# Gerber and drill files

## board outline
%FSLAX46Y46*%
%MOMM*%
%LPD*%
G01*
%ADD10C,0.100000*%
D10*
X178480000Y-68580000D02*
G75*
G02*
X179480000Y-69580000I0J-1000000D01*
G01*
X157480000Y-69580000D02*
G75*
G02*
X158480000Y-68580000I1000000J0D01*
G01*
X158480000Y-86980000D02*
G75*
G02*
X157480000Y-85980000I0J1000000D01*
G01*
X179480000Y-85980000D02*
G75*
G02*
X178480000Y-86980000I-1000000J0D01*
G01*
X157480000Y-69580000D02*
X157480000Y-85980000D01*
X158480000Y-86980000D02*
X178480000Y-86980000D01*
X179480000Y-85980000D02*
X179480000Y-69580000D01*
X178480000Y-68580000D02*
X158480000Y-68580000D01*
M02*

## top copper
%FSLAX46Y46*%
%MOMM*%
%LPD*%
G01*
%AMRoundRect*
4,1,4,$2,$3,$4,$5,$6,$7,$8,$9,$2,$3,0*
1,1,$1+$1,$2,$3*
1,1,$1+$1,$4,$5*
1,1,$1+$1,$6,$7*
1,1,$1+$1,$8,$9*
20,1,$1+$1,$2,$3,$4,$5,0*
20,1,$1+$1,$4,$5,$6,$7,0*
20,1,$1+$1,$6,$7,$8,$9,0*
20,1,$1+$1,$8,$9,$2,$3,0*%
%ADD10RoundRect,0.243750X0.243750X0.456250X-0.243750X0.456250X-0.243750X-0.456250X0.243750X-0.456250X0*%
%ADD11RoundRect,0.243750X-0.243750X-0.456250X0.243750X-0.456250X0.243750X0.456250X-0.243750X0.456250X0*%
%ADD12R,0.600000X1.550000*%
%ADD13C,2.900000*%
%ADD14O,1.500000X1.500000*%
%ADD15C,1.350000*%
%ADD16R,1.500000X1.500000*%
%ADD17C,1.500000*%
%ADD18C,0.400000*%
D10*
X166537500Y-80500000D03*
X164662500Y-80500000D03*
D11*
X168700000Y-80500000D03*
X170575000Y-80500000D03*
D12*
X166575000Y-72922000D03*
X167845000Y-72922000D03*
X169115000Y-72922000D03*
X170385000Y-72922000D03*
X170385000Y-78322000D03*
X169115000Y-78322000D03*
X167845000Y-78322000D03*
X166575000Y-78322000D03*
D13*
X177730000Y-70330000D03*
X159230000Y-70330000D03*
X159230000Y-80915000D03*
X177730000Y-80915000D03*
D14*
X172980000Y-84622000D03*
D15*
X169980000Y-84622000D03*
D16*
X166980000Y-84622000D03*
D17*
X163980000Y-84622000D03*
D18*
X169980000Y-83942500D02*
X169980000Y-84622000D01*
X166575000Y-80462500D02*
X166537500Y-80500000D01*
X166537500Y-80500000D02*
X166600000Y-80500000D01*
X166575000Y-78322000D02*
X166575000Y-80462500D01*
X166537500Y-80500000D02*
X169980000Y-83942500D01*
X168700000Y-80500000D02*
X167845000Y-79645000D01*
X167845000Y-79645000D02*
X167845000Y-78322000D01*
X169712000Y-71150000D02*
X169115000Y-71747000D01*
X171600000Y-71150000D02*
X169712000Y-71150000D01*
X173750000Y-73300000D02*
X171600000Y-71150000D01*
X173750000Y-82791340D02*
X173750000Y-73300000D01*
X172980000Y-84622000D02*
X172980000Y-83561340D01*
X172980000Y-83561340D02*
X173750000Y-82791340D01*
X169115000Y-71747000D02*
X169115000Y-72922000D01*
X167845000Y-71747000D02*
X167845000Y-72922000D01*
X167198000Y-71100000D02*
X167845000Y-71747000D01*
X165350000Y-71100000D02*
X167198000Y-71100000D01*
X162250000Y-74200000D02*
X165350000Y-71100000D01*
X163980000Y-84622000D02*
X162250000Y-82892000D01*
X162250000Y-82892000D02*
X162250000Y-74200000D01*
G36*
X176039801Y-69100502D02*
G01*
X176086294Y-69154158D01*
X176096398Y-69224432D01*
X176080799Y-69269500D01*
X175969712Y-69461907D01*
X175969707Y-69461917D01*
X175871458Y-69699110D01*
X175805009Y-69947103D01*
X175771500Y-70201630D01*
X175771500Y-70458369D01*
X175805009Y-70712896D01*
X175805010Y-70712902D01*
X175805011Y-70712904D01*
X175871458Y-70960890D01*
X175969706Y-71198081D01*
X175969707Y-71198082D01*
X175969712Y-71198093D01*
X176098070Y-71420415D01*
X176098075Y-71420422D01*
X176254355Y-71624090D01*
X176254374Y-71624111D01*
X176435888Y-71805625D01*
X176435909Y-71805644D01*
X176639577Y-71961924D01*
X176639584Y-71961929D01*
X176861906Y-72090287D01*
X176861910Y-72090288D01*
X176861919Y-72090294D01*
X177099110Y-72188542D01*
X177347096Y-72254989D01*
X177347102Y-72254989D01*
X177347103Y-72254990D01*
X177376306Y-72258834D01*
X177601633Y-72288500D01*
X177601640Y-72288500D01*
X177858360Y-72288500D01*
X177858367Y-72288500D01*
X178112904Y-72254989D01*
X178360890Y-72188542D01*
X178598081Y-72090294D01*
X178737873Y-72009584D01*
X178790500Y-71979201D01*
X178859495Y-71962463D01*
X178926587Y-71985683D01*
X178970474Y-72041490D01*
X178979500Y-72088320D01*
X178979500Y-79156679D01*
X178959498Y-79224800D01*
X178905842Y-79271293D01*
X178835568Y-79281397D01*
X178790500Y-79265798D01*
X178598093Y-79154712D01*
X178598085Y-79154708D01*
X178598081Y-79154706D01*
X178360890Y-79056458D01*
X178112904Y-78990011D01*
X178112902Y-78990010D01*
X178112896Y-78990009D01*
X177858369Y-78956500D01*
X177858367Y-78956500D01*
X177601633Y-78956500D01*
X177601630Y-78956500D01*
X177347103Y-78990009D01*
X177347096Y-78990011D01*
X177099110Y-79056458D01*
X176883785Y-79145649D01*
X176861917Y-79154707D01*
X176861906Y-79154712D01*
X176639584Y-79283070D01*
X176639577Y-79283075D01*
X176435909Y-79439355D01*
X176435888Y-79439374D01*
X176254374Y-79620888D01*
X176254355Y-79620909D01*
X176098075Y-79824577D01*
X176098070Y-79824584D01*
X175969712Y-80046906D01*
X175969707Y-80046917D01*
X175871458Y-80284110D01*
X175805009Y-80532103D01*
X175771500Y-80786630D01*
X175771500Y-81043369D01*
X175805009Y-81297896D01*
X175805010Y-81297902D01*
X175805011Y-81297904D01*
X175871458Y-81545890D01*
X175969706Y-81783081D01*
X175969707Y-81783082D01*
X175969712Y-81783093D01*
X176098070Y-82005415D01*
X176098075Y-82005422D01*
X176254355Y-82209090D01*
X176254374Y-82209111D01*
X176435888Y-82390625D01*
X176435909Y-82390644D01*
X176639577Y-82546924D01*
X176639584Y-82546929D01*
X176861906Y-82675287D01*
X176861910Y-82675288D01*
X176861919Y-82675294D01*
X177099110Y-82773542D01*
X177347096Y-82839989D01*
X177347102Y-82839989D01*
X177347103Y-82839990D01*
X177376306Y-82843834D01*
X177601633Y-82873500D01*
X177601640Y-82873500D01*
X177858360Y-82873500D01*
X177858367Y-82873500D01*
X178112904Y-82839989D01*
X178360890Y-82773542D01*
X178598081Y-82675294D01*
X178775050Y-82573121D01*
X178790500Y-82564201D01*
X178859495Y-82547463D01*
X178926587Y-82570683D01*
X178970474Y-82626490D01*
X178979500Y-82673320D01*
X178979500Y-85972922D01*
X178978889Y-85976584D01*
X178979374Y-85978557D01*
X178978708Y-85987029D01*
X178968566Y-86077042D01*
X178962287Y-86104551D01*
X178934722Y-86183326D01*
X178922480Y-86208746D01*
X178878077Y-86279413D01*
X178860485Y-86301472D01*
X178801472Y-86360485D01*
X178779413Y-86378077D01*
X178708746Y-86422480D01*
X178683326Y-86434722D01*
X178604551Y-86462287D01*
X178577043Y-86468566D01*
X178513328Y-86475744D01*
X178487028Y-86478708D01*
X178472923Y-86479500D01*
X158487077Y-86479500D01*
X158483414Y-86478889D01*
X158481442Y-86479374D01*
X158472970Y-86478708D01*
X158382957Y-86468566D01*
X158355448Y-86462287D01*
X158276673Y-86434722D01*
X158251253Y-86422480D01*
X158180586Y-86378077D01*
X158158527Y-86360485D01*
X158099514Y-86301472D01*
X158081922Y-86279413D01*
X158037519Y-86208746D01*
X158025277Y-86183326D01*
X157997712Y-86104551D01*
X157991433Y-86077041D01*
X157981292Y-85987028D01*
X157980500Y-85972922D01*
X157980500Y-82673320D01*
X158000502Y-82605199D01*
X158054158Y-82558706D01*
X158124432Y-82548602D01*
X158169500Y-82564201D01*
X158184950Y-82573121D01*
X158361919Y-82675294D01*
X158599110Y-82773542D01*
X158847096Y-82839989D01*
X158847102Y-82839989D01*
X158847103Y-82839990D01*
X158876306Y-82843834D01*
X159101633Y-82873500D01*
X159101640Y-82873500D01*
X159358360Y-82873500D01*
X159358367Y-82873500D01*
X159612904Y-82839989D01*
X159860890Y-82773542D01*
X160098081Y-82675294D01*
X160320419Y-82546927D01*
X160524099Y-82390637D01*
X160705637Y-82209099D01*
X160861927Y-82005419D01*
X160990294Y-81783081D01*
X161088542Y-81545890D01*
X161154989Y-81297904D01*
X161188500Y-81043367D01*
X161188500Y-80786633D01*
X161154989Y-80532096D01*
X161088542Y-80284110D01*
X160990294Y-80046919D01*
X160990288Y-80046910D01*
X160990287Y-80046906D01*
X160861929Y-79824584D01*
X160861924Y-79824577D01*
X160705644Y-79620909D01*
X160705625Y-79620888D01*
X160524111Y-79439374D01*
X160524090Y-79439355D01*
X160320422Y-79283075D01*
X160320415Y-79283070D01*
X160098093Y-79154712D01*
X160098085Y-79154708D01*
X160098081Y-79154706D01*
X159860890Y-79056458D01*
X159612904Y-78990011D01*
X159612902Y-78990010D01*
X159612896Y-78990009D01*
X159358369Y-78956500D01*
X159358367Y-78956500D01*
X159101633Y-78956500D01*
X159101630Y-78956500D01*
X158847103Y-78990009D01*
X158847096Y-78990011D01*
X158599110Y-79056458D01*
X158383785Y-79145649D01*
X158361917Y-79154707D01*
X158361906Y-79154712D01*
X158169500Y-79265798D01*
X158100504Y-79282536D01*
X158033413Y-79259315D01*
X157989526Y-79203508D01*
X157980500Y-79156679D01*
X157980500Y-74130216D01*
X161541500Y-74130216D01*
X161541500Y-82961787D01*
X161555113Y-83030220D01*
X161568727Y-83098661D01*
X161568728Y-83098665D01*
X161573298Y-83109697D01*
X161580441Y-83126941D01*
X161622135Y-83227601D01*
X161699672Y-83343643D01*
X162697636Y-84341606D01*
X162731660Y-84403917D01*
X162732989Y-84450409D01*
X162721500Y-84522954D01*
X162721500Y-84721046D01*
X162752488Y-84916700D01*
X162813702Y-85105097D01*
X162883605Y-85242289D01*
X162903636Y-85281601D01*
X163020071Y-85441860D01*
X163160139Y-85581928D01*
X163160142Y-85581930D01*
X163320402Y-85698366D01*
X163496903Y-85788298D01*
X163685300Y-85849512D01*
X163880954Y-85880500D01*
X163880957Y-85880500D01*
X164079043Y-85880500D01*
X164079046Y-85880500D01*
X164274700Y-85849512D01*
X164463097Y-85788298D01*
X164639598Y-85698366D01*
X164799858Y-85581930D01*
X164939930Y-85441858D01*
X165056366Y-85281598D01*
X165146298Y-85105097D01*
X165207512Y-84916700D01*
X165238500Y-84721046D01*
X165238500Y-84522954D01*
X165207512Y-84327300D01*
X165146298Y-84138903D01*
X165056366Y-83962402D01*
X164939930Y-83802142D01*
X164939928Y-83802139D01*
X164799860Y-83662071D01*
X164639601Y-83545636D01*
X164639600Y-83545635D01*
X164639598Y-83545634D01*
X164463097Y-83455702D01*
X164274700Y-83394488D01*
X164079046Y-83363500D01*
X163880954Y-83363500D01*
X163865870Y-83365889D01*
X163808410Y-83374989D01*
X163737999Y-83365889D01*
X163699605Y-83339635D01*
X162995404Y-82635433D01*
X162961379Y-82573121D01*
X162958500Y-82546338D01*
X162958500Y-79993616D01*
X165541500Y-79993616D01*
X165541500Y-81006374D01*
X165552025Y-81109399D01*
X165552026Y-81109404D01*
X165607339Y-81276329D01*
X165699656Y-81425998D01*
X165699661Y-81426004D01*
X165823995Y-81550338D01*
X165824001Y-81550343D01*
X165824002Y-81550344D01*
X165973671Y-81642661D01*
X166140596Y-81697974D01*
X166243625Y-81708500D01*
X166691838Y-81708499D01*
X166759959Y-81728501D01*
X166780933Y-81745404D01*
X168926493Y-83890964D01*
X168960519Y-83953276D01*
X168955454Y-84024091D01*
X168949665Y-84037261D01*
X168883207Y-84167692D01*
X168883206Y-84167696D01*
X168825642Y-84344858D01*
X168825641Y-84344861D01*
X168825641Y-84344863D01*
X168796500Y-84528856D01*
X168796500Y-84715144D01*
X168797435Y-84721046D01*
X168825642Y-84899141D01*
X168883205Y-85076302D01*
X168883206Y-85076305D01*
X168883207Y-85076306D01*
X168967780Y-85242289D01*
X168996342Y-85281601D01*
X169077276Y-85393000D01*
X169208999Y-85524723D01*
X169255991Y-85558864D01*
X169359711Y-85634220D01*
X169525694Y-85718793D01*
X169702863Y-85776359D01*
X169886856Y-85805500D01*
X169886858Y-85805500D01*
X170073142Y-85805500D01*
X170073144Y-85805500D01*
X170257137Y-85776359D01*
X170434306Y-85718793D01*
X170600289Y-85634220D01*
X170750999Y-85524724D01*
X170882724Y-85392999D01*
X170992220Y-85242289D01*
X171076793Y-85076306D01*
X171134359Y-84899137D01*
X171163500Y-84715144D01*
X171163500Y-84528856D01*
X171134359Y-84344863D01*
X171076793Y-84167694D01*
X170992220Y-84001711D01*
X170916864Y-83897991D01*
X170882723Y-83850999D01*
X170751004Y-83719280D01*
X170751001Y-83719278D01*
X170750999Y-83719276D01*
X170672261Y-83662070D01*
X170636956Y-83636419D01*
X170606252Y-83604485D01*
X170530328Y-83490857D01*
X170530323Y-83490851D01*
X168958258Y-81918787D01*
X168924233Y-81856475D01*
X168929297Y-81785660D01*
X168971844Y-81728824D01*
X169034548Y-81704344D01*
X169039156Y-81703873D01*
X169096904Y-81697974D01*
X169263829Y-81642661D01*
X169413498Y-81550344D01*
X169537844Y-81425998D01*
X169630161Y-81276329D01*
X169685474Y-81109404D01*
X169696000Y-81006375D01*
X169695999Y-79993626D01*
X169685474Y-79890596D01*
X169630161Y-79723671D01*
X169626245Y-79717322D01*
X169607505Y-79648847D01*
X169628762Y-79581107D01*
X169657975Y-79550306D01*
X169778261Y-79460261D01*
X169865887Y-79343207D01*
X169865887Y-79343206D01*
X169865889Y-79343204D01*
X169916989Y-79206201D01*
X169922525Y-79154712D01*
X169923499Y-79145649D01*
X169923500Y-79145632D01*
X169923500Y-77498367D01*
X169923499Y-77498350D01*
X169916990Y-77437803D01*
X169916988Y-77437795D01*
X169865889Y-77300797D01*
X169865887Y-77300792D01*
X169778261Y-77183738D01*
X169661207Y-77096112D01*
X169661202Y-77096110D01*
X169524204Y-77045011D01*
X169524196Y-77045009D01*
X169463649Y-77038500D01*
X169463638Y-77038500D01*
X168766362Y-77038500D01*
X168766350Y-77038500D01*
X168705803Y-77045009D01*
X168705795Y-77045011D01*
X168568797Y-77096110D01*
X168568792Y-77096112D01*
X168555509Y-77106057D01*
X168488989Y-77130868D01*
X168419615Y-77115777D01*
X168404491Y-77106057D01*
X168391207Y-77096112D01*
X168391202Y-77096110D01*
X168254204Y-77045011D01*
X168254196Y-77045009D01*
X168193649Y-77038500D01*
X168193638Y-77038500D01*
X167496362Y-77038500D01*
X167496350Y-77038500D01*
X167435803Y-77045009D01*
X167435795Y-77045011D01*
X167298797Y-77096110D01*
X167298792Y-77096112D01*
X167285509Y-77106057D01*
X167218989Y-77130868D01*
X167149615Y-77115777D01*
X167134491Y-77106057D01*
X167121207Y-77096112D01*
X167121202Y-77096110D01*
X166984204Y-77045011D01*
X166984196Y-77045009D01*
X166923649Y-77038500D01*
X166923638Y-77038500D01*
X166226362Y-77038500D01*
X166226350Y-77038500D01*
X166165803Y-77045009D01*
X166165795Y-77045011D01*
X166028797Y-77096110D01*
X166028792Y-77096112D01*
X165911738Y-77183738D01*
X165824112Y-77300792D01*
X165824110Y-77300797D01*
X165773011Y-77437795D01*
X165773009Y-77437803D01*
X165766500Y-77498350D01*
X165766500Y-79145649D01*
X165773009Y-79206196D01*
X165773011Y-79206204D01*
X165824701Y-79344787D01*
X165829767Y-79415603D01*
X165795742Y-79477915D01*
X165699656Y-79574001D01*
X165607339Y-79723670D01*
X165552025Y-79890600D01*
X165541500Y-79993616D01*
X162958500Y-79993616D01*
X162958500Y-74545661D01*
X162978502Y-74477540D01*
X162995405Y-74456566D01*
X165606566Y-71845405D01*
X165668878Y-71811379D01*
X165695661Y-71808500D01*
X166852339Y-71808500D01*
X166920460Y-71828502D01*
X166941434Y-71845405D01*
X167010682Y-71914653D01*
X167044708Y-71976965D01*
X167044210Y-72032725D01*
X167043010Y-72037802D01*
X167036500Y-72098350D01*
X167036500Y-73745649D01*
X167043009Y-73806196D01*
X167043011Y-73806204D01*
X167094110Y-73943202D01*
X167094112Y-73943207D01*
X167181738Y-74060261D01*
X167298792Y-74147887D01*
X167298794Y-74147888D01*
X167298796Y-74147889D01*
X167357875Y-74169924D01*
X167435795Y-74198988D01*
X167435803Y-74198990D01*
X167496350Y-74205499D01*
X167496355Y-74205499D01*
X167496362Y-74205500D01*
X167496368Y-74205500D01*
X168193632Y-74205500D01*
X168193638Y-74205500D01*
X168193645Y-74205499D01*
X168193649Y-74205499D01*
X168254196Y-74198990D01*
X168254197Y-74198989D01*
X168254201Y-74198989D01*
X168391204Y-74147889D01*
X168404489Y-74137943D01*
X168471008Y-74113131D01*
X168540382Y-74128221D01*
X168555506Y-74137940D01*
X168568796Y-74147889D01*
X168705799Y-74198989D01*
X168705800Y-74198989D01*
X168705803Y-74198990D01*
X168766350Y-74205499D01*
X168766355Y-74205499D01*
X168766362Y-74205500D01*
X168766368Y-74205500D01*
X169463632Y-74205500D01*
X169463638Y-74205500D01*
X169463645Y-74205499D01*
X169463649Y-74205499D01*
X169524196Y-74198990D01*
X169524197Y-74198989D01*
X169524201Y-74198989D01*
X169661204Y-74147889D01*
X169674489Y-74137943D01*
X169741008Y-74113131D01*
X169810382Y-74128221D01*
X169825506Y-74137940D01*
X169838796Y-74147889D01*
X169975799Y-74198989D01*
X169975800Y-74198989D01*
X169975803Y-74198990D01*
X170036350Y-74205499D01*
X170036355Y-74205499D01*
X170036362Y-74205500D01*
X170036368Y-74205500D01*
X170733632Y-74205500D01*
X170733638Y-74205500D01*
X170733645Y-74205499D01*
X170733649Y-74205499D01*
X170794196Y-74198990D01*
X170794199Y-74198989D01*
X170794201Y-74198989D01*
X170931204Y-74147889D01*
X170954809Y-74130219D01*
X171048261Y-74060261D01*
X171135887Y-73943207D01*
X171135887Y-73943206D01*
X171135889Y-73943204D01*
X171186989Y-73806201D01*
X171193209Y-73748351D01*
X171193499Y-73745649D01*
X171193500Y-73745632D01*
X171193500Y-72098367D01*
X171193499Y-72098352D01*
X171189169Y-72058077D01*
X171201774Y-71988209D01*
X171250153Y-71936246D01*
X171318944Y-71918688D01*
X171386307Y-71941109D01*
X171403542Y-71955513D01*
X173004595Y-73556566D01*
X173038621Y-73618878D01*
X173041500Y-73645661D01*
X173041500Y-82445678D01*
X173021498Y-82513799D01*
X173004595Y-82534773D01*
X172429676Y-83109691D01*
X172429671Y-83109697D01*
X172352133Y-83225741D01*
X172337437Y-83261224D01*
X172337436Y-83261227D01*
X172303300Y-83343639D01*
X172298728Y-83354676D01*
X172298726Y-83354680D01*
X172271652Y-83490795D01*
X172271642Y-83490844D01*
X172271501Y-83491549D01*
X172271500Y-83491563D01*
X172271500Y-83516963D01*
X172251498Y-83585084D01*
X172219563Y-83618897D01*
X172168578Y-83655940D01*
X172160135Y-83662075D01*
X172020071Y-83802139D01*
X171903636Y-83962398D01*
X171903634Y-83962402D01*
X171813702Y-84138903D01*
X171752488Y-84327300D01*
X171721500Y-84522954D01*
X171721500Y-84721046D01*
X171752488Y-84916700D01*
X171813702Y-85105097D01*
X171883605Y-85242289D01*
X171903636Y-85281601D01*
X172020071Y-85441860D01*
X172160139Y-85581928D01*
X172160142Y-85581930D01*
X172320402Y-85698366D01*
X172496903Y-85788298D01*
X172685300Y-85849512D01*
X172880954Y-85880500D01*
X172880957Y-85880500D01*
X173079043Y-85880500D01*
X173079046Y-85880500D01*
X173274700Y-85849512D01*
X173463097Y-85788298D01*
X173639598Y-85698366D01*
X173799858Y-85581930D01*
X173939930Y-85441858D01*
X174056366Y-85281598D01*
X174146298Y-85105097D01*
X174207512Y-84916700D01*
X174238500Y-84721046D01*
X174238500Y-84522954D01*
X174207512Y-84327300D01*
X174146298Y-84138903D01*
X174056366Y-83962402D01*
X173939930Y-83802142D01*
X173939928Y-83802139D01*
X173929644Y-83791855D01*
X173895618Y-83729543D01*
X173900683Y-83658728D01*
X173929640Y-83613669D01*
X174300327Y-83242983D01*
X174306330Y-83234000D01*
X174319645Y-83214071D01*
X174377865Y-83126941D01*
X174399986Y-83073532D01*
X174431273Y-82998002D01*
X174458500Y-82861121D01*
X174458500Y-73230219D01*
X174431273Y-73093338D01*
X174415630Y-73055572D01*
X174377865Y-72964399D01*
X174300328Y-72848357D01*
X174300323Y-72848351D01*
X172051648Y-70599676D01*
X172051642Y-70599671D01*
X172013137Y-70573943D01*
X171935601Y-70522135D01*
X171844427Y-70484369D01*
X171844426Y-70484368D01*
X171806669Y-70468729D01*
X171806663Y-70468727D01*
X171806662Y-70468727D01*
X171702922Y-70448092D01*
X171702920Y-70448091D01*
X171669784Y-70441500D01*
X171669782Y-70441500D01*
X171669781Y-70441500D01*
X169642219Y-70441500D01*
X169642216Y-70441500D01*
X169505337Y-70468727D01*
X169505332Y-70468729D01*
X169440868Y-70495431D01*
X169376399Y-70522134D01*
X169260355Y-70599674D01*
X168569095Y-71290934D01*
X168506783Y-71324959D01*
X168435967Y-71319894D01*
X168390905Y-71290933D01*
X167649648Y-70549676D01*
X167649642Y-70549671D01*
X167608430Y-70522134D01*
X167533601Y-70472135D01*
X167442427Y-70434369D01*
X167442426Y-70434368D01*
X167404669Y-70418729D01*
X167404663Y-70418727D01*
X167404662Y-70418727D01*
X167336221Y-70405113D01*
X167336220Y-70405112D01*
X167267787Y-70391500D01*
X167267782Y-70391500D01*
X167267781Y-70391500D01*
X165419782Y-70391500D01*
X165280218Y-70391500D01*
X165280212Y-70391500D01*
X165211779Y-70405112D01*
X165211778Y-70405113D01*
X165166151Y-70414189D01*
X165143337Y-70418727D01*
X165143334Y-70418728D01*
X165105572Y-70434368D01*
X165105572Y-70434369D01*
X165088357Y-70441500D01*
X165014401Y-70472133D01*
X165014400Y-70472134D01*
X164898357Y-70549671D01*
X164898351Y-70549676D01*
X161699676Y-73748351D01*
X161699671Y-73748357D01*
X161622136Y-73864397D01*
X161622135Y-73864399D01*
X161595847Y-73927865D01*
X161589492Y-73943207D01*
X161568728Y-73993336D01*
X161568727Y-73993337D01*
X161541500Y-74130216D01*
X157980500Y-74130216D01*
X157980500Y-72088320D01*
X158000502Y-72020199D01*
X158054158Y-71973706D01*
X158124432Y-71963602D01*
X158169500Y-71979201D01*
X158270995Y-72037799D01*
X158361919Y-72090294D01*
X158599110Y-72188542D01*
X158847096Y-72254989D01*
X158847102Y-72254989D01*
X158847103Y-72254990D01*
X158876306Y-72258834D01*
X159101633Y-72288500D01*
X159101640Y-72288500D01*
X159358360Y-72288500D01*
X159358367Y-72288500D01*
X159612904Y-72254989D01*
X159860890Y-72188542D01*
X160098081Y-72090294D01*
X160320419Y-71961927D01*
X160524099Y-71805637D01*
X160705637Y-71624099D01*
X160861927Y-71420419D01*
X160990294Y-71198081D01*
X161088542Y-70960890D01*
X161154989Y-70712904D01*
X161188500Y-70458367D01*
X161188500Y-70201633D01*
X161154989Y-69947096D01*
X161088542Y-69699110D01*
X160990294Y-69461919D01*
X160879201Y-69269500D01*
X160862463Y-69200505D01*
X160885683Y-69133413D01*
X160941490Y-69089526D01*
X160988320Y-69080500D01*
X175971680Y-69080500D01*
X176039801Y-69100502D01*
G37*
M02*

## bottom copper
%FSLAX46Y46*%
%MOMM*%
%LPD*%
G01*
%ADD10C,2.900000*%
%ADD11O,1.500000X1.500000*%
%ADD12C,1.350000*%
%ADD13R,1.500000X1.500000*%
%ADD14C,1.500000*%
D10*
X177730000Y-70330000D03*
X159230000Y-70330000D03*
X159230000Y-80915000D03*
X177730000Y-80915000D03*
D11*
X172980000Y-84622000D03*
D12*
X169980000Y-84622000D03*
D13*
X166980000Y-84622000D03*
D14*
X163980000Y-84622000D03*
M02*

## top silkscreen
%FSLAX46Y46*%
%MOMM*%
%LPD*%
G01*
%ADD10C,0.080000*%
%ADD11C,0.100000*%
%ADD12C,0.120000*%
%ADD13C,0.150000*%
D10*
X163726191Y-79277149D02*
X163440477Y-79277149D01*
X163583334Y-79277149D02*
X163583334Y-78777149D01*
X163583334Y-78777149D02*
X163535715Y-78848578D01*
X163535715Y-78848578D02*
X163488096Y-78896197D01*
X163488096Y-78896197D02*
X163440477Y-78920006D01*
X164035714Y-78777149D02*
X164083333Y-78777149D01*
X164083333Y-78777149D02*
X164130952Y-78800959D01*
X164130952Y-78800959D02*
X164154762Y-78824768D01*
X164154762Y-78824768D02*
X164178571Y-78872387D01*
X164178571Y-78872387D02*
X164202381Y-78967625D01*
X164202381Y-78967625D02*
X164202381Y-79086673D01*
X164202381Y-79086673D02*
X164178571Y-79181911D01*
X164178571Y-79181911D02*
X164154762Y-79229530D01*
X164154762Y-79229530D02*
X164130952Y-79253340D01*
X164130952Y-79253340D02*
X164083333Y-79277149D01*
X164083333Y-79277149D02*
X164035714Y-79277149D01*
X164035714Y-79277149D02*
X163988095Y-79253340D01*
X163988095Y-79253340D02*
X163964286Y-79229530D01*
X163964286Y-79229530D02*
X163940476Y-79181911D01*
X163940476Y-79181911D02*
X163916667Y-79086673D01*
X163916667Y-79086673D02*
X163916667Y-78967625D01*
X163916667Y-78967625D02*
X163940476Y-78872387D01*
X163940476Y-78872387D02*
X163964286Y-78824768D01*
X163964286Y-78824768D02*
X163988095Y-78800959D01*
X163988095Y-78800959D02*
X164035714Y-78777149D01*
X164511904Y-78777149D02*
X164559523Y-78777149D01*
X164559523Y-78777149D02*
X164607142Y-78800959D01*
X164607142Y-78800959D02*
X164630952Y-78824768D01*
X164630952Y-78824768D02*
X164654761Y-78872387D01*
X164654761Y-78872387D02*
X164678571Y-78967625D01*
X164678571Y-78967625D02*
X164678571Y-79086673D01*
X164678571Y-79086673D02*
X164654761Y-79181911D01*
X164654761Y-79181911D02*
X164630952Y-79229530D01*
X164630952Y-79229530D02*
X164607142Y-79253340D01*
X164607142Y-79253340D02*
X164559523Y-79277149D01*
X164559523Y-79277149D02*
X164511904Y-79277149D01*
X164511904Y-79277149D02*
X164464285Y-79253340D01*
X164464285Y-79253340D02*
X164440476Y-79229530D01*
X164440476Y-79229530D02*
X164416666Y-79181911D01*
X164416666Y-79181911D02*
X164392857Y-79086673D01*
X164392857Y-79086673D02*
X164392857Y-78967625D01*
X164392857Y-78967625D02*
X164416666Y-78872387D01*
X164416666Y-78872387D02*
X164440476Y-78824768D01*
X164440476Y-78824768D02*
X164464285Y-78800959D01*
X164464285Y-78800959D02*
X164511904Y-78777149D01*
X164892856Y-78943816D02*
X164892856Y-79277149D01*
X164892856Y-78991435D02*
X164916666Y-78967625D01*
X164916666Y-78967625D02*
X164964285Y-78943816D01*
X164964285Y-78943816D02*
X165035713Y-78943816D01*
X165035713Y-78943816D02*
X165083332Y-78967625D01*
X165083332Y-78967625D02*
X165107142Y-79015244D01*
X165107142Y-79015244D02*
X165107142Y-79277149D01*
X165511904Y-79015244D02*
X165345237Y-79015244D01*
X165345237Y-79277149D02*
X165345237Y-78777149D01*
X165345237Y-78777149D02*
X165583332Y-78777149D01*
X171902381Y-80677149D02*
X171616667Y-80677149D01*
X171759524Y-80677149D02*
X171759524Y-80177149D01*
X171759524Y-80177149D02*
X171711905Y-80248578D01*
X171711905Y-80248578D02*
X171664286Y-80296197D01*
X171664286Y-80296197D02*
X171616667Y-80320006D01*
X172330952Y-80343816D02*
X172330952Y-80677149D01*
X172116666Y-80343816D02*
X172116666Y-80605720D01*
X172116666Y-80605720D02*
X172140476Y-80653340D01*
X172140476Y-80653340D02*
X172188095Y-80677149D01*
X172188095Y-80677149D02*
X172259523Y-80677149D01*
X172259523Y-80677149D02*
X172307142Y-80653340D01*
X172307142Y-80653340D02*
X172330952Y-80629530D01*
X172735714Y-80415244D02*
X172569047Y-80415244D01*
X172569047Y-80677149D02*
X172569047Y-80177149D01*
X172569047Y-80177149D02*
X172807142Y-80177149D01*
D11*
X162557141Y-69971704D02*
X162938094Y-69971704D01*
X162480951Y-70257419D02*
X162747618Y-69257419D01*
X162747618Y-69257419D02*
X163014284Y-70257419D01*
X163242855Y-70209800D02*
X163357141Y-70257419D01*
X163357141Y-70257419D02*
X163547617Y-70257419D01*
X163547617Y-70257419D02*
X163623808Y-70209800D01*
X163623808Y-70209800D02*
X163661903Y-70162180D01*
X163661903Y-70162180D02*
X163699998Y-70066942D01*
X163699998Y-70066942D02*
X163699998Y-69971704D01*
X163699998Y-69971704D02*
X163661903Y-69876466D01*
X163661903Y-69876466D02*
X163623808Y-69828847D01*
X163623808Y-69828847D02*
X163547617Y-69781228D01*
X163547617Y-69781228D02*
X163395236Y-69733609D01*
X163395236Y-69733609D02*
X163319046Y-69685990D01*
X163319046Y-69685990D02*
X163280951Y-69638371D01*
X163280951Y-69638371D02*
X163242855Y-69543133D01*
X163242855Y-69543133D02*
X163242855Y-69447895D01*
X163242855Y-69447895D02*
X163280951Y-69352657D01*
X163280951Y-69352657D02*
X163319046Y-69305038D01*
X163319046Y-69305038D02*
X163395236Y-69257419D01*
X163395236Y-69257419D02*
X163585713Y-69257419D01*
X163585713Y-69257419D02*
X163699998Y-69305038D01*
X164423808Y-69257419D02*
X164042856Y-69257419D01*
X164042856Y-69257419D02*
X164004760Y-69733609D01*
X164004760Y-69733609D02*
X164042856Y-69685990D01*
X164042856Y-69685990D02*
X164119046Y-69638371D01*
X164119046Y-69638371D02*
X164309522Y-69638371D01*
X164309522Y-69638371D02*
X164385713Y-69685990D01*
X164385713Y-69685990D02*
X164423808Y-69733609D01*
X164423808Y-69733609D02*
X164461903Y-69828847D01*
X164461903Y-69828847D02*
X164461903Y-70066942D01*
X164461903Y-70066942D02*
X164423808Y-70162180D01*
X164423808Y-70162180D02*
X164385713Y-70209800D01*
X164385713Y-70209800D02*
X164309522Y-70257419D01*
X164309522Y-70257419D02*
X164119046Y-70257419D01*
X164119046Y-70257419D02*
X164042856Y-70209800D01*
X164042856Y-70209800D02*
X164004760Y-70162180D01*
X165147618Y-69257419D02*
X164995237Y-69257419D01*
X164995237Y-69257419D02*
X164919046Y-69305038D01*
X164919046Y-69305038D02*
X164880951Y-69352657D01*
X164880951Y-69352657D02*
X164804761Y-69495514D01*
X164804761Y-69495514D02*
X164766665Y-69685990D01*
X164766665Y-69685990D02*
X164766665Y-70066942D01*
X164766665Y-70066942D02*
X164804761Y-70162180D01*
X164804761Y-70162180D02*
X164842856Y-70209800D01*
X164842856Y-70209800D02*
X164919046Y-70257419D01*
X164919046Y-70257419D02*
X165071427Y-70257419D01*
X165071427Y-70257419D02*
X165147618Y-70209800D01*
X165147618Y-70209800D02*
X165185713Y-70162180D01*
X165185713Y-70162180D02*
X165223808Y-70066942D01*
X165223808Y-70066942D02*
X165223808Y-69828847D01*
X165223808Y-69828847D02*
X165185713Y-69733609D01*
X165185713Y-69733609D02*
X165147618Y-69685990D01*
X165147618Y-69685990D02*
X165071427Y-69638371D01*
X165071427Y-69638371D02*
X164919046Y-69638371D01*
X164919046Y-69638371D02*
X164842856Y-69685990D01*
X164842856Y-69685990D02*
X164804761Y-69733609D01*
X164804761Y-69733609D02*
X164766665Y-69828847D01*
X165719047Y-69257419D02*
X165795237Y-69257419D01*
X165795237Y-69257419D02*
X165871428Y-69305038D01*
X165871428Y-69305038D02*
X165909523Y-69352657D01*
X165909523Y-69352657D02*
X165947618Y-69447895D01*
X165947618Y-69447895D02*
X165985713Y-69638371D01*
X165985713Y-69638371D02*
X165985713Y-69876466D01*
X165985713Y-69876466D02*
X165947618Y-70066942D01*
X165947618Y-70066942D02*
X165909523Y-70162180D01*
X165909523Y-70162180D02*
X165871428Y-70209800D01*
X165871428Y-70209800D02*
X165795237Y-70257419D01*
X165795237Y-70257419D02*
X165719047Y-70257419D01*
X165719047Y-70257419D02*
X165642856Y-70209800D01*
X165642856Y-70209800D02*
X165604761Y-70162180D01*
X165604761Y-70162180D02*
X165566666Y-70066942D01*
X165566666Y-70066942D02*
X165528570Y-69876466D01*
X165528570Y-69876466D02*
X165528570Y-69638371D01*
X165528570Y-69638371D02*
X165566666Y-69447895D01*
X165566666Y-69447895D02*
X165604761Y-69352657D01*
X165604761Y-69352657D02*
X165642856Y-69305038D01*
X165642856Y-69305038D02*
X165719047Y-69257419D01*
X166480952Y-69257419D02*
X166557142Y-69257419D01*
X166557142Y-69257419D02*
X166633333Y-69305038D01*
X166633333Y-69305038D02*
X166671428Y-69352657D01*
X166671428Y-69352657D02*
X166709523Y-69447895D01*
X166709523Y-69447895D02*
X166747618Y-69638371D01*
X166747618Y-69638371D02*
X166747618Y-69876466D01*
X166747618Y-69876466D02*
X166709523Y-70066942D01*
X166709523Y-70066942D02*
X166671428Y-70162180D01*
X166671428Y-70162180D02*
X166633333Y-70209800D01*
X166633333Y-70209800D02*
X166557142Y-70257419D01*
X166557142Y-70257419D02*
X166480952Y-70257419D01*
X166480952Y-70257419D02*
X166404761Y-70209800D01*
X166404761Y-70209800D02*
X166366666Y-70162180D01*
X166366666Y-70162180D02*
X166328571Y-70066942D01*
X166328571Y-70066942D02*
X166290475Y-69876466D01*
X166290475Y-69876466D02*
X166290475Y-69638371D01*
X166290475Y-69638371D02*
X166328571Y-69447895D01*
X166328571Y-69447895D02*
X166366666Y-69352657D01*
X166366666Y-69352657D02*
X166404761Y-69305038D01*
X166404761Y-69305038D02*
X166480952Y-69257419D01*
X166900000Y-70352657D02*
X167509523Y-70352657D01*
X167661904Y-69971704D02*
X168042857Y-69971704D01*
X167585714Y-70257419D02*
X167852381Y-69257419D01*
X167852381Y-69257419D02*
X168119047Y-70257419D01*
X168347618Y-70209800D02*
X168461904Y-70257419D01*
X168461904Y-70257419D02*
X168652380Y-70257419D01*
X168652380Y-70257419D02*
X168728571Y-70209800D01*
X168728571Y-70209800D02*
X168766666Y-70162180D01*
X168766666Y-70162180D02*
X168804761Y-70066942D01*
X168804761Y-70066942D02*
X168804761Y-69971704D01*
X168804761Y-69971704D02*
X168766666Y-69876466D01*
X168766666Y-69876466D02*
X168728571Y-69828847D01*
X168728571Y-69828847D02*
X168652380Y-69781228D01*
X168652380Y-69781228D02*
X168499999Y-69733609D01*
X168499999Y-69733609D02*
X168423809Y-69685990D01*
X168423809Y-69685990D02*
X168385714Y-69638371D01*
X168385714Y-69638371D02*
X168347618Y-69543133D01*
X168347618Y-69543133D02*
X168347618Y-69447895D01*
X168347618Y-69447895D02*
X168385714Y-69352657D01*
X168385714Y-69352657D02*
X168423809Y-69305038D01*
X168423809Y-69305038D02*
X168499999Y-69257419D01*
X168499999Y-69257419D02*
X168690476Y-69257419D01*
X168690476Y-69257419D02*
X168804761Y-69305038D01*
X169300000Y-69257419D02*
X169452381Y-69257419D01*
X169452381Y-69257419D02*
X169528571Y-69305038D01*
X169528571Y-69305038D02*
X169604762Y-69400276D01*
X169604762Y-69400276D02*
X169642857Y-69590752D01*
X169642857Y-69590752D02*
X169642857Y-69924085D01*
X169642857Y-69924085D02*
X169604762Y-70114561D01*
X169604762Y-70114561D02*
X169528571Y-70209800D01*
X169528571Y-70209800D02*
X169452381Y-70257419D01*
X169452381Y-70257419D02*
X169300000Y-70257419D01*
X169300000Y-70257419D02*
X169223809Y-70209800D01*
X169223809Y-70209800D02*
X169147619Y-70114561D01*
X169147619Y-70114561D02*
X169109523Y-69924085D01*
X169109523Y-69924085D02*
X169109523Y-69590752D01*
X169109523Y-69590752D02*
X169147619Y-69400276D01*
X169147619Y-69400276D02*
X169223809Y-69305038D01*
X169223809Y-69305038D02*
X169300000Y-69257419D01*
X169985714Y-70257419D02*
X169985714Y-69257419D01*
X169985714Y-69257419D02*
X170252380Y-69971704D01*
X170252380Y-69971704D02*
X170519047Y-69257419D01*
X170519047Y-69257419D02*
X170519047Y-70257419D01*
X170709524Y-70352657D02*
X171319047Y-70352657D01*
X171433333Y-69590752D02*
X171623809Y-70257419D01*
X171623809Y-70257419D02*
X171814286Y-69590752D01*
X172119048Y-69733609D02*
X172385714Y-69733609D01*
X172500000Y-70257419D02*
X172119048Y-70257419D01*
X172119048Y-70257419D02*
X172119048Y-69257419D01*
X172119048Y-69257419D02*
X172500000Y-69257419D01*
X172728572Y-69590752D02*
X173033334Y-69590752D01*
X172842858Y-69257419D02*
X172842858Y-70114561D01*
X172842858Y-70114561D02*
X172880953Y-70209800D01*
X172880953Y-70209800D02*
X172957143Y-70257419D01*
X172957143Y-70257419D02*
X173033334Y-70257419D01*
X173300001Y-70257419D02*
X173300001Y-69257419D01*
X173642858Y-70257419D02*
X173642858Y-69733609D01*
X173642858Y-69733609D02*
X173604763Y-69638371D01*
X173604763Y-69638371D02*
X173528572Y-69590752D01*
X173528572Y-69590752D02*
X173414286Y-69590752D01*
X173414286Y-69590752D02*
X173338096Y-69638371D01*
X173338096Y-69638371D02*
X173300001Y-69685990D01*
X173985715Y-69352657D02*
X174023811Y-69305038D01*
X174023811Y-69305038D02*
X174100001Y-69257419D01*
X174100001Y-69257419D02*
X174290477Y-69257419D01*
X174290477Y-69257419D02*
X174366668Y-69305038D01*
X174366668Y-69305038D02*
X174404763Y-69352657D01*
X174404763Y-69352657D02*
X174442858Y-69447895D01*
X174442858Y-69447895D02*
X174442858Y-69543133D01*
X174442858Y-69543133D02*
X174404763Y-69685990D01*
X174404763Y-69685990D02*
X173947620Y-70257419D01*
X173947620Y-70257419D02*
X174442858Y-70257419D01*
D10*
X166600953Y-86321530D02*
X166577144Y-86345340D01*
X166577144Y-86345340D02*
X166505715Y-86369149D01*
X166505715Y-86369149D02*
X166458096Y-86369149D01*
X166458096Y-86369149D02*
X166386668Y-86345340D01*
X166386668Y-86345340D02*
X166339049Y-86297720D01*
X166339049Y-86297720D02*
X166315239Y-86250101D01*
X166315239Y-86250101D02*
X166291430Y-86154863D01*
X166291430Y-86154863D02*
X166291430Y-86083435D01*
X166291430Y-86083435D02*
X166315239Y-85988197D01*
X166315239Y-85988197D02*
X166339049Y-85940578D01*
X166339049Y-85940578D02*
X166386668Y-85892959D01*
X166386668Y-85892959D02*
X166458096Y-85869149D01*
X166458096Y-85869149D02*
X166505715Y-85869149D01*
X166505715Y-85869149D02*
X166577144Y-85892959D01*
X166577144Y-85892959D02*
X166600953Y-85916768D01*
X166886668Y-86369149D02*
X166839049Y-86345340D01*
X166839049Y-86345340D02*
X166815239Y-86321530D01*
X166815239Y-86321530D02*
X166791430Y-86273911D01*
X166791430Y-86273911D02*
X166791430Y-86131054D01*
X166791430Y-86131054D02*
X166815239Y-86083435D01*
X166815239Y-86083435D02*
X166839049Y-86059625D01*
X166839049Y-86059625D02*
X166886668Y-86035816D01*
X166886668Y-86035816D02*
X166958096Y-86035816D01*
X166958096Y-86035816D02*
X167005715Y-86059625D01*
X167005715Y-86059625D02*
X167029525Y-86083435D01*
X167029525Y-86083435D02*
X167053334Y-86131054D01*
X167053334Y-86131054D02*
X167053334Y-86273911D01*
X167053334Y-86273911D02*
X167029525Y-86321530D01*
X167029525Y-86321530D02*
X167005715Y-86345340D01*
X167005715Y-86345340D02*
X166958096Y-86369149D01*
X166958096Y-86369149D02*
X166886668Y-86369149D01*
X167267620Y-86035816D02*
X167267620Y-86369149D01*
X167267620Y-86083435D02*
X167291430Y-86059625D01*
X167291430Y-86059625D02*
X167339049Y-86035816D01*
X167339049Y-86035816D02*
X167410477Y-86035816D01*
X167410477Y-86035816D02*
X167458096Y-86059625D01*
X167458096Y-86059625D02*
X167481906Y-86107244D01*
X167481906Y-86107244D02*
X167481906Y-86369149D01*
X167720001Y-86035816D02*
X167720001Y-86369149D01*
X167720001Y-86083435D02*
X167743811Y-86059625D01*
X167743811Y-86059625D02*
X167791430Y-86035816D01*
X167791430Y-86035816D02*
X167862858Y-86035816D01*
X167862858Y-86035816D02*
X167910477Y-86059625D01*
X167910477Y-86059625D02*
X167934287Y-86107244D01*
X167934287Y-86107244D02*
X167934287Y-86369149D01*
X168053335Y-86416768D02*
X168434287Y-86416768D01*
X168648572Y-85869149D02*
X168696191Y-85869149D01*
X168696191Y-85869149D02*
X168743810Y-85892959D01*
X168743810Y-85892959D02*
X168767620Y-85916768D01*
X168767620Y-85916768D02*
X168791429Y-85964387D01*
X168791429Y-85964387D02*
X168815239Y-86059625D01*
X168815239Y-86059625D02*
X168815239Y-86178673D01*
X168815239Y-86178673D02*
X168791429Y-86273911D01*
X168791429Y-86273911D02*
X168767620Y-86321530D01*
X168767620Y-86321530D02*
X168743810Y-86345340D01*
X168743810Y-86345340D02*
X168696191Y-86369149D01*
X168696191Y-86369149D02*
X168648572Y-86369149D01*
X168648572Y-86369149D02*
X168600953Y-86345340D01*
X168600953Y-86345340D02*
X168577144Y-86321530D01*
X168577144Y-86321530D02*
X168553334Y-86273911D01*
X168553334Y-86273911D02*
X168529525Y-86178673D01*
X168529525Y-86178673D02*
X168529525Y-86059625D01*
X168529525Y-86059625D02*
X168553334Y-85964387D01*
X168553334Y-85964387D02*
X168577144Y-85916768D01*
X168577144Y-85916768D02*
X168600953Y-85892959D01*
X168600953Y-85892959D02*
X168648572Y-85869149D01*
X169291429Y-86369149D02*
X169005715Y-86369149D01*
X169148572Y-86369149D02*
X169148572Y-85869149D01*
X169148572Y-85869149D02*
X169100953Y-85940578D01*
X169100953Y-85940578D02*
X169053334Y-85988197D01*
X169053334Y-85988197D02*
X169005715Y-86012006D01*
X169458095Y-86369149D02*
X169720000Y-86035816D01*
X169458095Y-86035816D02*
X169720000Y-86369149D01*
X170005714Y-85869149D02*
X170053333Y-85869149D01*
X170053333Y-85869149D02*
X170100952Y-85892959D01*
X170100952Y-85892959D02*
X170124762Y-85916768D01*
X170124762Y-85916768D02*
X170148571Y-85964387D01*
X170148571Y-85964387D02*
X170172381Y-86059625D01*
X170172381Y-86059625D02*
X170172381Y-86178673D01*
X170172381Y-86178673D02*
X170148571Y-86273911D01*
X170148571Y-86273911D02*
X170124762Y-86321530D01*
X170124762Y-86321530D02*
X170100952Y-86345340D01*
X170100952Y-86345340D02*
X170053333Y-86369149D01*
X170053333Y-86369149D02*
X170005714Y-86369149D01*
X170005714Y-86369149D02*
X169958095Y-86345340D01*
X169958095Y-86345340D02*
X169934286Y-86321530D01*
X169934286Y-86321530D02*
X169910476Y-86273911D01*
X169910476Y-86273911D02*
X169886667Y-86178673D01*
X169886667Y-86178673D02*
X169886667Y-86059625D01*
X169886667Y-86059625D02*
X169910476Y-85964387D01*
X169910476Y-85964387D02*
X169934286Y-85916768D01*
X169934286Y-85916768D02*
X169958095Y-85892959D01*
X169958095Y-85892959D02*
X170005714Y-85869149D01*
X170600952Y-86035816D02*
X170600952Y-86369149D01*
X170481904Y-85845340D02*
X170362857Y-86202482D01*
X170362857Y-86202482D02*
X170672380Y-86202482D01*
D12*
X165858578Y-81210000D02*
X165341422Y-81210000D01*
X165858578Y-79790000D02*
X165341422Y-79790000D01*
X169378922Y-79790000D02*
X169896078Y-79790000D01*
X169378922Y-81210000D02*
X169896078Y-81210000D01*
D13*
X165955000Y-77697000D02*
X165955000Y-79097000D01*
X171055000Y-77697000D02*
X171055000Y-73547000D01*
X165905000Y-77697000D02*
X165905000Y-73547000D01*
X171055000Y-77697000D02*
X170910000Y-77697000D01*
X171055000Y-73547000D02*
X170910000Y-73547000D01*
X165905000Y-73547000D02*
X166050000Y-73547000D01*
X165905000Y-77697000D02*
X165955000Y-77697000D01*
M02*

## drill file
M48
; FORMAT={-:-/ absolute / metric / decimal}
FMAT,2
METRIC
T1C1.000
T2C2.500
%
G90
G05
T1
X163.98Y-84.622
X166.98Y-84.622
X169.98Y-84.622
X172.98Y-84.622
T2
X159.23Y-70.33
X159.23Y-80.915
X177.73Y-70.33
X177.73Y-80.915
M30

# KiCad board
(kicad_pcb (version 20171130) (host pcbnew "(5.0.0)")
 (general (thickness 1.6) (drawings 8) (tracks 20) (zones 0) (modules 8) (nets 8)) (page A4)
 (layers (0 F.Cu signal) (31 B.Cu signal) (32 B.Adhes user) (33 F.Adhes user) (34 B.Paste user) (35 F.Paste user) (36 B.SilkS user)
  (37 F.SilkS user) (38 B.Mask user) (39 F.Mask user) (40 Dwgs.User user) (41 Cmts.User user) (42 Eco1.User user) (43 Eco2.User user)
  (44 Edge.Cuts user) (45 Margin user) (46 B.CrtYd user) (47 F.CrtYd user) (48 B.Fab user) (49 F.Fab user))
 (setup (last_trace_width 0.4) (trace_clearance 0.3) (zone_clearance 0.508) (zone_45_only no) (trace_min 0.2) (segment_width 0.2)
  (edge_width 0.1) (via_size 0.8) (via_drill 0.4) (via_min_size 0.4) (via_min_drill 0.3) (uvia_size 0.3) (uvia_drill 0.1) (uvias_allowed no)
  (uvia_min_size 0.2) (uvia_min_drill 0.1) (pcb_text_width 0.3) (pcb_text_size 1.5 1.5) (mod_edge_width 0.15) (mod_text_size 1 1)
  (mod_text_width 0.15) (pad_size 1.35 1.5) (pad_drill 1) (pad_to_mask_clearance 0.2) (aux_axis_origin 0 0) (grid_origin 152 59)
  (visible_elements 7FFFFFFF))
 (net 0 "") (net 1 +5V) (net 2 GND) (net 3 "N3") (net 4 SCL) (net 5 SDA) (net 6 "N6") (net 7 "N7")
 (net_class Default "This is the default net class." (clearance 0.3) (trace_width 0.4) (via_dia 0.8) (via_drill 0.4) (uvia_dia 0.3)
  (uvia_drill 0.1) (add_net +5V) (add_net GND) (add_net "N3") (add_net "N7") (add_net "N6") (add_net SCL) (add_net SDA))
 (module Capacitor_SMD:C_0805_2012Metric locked (layer F.Cu) (at 165.6 80.5 180)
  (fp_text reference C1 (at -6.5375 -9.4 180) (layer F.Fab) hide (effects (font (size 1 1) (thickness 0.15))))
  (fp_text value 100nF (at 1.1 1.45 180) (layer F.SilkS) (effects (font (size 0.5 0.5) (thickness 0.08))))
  (fp_line (start -0.258578 -0.71) (end 0.258578 -0.71) (layer F.SilkS) (width 0.12))
  (fp_line (start -0.258578 0.71) (end 0.258578 0.71) (layer F.SilkS) (width 0.12))
  (pad 1 smd roundrect (at -0.9375 0 180) (size 0.975 1.4) (layers F.Cu F.Paste F.Mask) (roundrect_rratio 0.25) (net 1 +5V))
  (pad 2 smd roundrect (at 0.9375 0 180) (size 0.975 1.4) (layers F.Cu F.Paste F.Mask) (roundrect_rratio 0.25) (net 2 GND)))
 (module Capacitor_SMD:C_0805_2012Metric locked (layer F.Cu) (at 169.6375 80.5)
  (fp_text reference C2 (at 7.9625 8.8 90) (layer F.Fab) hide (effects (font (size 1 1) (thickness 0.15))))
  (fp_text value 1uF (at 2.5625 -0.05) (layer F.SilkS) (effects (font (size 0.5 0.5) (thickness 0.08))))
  (fp_line (start -0.258578 -0.71) (end 0.258578 -0.71) (layer F.SilkS) (width 0.12))
  (fp_line (start -0.258578 0.71) (end 0.258578 0.71) (layer F.SilkS) (width 0.12))
  (pad 1 smd roundrect (at -0.9375 0) (size 0.975 1.4) (layers F.Cu F.Paste F.Mask) (roundrect_rratio 0.25) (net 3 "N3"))
  (pad 2 smd roundrect (at 0.9375 0) (size 0.975 1.4) (layers F.Cu F.Paste F.Mask) (roundrect_rratio 0.25) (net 2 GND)))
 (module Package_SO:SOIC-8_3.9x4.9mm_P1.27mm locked (layer F.Cu) (at 168.48 75.622 90)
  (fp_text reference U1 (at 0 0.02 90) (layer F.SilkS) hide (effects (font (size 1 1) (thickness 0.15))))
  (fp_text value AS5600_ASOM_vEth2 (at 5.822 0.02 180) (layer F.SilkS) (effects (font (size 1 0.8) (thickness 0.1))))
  (fp_line (start -2.075 -2.525) (end -3.475 -2.525) (layer F.SilkS) (width 0.15))
  (fp_line (start -2.075 2.575) (end 2.075 2.575) (layer F.SilkS) (width 0.15))
  (fp_line (start -2.075 -2.575) (end 2.075 -2.575) (layer F.SilkS) (width 0.15))
  (fp_line (start -2.075 2.575) (end -2.075 2.43) (layer F.SilkS) (width 0.15))
  (fp_line (start 2.075 2.575) (end 2.075 2.43) (layer F.SilkS) (width 0.15))
  (fp_line (start 2.075 -2.575) (end 2.075 -2.43) (layer F.SilkS) (width 0.15))
  (fp_line (start -2.075 -2.575) (end -2.075 -2.525) (layer F.SilkS) (width 0.15))
  (pad 8 smd rect (at 2.7 -1.905 90) (size 1.55 0.6) (layers F.Cu F.Paste F.Mask) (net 2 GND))
  (pad 7 smd rect (at 2.7 -0.635 90) (size 1.55 0.6) (layers F.Cu F.Paste F.Mask) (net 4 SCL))
  (pad 6 smd rect (at 2.7 0.635 90) (size 1.55 0.6) (layers F.Cu F.Paste F.Mask) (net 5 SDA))
  (pad 5 smd rect (at 2.7 1.905 90) (size 1.55 0.6) (layers F.Cu F.Paste F.Mask) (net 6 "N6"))
  (pad 4 smd rect (at -2.7 1.905 90) (size 1.55 0.6) (layers F.Cu F.Paste F.Mask) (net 2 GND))
  (pad 3 smd rect (at -2.7 0.635 90) (size 1.55 0.6) (layers F.Cu F.Paste F.Mask) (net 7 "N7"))
  (pad 2 smd rect (at -2.7 -0.635 90) (size 1.55 0.6) (layers F.Cu F.Paste F.Mask) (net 3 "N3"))
  (pad 1 smd rect (at -2.7 -1.905 90) (size 1.55 0.6) (layers F.Cu F.Paste F.Mask) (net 1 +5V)))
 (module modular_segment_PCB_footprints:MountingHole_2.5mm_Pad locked (layer F.Cu) (at 177.73 70.33)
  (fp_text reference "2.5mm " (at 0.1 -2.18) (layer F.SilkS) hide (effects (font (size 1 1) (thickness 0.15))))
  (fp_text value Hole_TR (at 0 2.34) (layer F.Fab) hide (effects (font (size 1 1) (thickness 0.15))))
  (pad "" np_thru_hole circle (at 0 0) (size 2.9 2.9) (drill 2.5) (layers *.Cu *.Mask)))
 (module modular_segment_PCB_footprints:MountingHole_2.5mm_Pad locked (layer F.Cu) (at 159.23 70.33)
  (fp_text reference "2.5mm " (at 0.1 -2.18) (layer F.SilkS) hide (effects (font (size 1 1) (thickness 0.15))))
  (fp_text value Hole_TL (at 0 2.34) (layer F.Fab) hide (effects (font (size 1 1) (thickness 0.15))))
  (pad "" np_thru_hole circle (at 0 0) (size 2.9 2.9) (drill 2.5) (layers *.Cu *.Mask)))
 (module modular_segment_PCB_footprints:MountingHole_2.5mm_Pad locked (layer F.Cu) (at 159.23 80.915)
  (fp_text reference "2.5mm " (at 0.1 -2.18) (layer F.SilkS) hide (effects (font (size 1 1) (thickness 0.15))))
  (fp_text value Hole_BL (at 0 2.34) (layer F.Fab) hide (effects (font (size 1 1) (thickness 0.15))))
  (pad "" np_thru_hole circle (at 0 0) (size 2.9 2.9) (drill 2.5) (layers *.Cu *.Mask)))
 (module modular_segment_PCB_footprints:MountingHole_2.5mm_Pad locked (layer F.Cu) (at 177.73 80.915)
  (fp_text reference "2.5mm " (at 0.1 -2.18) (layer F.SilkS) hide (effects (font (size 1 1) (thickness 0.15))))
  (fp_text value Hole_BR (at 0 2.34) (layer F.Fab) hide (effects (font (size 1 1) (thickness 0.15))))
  (pad "" np_thru_hole circle (at 0 0) (size 2.9 2.9) (drill 2.5) (layers *.Cu *.Mask)))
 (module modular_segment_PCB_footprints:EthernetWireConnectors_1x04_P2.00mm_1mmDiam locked (layer F.Cu) (at 168.48 84.622)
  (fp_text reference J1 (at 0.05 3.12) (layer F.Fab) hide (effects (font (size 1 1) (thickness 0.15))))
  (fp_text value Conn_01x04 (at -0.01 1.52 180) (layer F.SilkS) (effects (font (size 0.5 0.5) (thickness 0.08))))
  (pad 4 thru_hole oval (at 4.5 0 90) (size 1.5 1.5) (drill 1) (layers *.Cu *.Mask) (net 5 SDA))
  (pad 3 thru_hole circle (at 1.5 0 90) (size 1.35 1.35) (drill 1) (layers *.Cu *.Mask) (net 1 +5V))
  (pad 2 thru_hole rect (at -1.5 0 90) (size 1.5 1.5) (drill 1) (layers *.Cu *.Mask) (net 2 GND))
  (pad 1 thru_hole circle (at -4.5 0 90) (size 1.5 1.5) (drill 1) (layers *.Cu *.Mask) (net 4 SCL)))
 (gr_arc (start 178.48 69.58) (end 179.48 69.58) (angle -90) (layer Edge.Cuts) (width 0.1))
 (gr_arc (start 158.48 69.58) (end 158.48 68.58) (angle -90) (layer Edge.Cuts) (width 0.1))
 (gr_arc (start 158.48 85.98) (end 157.48 85.98) (angle -90) (layer Edge.Cuts) (width 0.1))
 (gr_arc (start 178.48 85.98) (end 178.48 86.98) (angle -90) (layer Edge.Cuts) (width 0.1))
 (gr_line (start 157.48 69.58) (end 157.48 85.98) (layer Edge.Cuts) (width 0.1))
 (gr_line (start 158.48 86.98) (end 178.48 86.98) (layer Edge.Cuts) (width 0.1))
 (gr_line (start 179.48 85.98) (end 179.48 69.58) (layer Edge.Cuts) (width 0.1))
 (gr_line (start 178.48 68.58) (end 158.48 68.58) (layer Edge.Cuts) (width 0.1))
 (segment (start 169.98 83.9425) (end 169.98 84.622) (width 0.4) (layer F.Cu) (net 1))
 (segment (start 166.575 80.4625) (end 166.5375 80.5) (width 0.4) (layer F.Cu) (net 1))
 (segment (start 166.5375 80.5) (end 166.6 80.5) (width 0.4) (layer F.Cu) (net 1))
 (segment (start 166.575 78.322) (end 166.575 80.4625) (width 0.4) (layer F.Cu) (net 1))
 (segment (start 166.5375 80.5) (end 169.98 83.9425) (width 0.4) (layer F.Cu) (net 1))
 (segment (start 168.7 80.5) (end 167.845 79.645) (width 0.4) (layer F.Cu) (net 3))
 (segment (start 167.845 79.645) (end 167.845 78.322) (width 0.4) (layer F.Cu) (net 3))
 (segment (start 169.712 71.15) (end 169.115 71.747) (width 0.4) (layer F.Cu) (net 5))
 (segment (start 171.6 71.15) (end 169.712 71.15) (width 0.4) (layer F.Cu) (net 5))
 (segment (start 173.75 73.3) (end 171.6 71.15) (width 0.4) (layer F.Cu) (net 5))
 (segment (start 173.75 82.79134) (end 173.75 73.3) (width 0.4) (layer F.Cu) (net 5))
 (segment (start 172.98 84.622) (end 172.98 83.56134) (width 0.4) (layer F.Cu) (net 5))
 (segment (start 172.98 83.56134) (end 173.75 82.79134) (width 0.4) (layer F.Cu) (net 5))
 (segment (start 169.115 71.747) (end 169.115 72.922) (width 0.4) (layer F.Cu) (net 5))
 (segment (start 167.845 71.747) (end 167.845 72.922) (width 0.4) (layer F.Cu) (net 4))
 (segment (start 167.198 71.1) (end 167.845 71.747) (width 0.4) (layer F.Cu) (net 4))
 (segment (start 165.35 71.1) (end 167.198 71.1) (width 0.4) (layer F.Cu) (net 4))
 (segment (start 162.25 74.2) (end 165.35 71.1) (width 0.4) (layer F.Cu) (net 4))
 (segment (start 163.98 84.622) (end 162.25 82.892) (width 0.4) (layer F.Cu) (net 4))
 (segment (start 162.25 82.892) (end 162.25 74.2) (width 0.4) (layer F.Cu) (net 4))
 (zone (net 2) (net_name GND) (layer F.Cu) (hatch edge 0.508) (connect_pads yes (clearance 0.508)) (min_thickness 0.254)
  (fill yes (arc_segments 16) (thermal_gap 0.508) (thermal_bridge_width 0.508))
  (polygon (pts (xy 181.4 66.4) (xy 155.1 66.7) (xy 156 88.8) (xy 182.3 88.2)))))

